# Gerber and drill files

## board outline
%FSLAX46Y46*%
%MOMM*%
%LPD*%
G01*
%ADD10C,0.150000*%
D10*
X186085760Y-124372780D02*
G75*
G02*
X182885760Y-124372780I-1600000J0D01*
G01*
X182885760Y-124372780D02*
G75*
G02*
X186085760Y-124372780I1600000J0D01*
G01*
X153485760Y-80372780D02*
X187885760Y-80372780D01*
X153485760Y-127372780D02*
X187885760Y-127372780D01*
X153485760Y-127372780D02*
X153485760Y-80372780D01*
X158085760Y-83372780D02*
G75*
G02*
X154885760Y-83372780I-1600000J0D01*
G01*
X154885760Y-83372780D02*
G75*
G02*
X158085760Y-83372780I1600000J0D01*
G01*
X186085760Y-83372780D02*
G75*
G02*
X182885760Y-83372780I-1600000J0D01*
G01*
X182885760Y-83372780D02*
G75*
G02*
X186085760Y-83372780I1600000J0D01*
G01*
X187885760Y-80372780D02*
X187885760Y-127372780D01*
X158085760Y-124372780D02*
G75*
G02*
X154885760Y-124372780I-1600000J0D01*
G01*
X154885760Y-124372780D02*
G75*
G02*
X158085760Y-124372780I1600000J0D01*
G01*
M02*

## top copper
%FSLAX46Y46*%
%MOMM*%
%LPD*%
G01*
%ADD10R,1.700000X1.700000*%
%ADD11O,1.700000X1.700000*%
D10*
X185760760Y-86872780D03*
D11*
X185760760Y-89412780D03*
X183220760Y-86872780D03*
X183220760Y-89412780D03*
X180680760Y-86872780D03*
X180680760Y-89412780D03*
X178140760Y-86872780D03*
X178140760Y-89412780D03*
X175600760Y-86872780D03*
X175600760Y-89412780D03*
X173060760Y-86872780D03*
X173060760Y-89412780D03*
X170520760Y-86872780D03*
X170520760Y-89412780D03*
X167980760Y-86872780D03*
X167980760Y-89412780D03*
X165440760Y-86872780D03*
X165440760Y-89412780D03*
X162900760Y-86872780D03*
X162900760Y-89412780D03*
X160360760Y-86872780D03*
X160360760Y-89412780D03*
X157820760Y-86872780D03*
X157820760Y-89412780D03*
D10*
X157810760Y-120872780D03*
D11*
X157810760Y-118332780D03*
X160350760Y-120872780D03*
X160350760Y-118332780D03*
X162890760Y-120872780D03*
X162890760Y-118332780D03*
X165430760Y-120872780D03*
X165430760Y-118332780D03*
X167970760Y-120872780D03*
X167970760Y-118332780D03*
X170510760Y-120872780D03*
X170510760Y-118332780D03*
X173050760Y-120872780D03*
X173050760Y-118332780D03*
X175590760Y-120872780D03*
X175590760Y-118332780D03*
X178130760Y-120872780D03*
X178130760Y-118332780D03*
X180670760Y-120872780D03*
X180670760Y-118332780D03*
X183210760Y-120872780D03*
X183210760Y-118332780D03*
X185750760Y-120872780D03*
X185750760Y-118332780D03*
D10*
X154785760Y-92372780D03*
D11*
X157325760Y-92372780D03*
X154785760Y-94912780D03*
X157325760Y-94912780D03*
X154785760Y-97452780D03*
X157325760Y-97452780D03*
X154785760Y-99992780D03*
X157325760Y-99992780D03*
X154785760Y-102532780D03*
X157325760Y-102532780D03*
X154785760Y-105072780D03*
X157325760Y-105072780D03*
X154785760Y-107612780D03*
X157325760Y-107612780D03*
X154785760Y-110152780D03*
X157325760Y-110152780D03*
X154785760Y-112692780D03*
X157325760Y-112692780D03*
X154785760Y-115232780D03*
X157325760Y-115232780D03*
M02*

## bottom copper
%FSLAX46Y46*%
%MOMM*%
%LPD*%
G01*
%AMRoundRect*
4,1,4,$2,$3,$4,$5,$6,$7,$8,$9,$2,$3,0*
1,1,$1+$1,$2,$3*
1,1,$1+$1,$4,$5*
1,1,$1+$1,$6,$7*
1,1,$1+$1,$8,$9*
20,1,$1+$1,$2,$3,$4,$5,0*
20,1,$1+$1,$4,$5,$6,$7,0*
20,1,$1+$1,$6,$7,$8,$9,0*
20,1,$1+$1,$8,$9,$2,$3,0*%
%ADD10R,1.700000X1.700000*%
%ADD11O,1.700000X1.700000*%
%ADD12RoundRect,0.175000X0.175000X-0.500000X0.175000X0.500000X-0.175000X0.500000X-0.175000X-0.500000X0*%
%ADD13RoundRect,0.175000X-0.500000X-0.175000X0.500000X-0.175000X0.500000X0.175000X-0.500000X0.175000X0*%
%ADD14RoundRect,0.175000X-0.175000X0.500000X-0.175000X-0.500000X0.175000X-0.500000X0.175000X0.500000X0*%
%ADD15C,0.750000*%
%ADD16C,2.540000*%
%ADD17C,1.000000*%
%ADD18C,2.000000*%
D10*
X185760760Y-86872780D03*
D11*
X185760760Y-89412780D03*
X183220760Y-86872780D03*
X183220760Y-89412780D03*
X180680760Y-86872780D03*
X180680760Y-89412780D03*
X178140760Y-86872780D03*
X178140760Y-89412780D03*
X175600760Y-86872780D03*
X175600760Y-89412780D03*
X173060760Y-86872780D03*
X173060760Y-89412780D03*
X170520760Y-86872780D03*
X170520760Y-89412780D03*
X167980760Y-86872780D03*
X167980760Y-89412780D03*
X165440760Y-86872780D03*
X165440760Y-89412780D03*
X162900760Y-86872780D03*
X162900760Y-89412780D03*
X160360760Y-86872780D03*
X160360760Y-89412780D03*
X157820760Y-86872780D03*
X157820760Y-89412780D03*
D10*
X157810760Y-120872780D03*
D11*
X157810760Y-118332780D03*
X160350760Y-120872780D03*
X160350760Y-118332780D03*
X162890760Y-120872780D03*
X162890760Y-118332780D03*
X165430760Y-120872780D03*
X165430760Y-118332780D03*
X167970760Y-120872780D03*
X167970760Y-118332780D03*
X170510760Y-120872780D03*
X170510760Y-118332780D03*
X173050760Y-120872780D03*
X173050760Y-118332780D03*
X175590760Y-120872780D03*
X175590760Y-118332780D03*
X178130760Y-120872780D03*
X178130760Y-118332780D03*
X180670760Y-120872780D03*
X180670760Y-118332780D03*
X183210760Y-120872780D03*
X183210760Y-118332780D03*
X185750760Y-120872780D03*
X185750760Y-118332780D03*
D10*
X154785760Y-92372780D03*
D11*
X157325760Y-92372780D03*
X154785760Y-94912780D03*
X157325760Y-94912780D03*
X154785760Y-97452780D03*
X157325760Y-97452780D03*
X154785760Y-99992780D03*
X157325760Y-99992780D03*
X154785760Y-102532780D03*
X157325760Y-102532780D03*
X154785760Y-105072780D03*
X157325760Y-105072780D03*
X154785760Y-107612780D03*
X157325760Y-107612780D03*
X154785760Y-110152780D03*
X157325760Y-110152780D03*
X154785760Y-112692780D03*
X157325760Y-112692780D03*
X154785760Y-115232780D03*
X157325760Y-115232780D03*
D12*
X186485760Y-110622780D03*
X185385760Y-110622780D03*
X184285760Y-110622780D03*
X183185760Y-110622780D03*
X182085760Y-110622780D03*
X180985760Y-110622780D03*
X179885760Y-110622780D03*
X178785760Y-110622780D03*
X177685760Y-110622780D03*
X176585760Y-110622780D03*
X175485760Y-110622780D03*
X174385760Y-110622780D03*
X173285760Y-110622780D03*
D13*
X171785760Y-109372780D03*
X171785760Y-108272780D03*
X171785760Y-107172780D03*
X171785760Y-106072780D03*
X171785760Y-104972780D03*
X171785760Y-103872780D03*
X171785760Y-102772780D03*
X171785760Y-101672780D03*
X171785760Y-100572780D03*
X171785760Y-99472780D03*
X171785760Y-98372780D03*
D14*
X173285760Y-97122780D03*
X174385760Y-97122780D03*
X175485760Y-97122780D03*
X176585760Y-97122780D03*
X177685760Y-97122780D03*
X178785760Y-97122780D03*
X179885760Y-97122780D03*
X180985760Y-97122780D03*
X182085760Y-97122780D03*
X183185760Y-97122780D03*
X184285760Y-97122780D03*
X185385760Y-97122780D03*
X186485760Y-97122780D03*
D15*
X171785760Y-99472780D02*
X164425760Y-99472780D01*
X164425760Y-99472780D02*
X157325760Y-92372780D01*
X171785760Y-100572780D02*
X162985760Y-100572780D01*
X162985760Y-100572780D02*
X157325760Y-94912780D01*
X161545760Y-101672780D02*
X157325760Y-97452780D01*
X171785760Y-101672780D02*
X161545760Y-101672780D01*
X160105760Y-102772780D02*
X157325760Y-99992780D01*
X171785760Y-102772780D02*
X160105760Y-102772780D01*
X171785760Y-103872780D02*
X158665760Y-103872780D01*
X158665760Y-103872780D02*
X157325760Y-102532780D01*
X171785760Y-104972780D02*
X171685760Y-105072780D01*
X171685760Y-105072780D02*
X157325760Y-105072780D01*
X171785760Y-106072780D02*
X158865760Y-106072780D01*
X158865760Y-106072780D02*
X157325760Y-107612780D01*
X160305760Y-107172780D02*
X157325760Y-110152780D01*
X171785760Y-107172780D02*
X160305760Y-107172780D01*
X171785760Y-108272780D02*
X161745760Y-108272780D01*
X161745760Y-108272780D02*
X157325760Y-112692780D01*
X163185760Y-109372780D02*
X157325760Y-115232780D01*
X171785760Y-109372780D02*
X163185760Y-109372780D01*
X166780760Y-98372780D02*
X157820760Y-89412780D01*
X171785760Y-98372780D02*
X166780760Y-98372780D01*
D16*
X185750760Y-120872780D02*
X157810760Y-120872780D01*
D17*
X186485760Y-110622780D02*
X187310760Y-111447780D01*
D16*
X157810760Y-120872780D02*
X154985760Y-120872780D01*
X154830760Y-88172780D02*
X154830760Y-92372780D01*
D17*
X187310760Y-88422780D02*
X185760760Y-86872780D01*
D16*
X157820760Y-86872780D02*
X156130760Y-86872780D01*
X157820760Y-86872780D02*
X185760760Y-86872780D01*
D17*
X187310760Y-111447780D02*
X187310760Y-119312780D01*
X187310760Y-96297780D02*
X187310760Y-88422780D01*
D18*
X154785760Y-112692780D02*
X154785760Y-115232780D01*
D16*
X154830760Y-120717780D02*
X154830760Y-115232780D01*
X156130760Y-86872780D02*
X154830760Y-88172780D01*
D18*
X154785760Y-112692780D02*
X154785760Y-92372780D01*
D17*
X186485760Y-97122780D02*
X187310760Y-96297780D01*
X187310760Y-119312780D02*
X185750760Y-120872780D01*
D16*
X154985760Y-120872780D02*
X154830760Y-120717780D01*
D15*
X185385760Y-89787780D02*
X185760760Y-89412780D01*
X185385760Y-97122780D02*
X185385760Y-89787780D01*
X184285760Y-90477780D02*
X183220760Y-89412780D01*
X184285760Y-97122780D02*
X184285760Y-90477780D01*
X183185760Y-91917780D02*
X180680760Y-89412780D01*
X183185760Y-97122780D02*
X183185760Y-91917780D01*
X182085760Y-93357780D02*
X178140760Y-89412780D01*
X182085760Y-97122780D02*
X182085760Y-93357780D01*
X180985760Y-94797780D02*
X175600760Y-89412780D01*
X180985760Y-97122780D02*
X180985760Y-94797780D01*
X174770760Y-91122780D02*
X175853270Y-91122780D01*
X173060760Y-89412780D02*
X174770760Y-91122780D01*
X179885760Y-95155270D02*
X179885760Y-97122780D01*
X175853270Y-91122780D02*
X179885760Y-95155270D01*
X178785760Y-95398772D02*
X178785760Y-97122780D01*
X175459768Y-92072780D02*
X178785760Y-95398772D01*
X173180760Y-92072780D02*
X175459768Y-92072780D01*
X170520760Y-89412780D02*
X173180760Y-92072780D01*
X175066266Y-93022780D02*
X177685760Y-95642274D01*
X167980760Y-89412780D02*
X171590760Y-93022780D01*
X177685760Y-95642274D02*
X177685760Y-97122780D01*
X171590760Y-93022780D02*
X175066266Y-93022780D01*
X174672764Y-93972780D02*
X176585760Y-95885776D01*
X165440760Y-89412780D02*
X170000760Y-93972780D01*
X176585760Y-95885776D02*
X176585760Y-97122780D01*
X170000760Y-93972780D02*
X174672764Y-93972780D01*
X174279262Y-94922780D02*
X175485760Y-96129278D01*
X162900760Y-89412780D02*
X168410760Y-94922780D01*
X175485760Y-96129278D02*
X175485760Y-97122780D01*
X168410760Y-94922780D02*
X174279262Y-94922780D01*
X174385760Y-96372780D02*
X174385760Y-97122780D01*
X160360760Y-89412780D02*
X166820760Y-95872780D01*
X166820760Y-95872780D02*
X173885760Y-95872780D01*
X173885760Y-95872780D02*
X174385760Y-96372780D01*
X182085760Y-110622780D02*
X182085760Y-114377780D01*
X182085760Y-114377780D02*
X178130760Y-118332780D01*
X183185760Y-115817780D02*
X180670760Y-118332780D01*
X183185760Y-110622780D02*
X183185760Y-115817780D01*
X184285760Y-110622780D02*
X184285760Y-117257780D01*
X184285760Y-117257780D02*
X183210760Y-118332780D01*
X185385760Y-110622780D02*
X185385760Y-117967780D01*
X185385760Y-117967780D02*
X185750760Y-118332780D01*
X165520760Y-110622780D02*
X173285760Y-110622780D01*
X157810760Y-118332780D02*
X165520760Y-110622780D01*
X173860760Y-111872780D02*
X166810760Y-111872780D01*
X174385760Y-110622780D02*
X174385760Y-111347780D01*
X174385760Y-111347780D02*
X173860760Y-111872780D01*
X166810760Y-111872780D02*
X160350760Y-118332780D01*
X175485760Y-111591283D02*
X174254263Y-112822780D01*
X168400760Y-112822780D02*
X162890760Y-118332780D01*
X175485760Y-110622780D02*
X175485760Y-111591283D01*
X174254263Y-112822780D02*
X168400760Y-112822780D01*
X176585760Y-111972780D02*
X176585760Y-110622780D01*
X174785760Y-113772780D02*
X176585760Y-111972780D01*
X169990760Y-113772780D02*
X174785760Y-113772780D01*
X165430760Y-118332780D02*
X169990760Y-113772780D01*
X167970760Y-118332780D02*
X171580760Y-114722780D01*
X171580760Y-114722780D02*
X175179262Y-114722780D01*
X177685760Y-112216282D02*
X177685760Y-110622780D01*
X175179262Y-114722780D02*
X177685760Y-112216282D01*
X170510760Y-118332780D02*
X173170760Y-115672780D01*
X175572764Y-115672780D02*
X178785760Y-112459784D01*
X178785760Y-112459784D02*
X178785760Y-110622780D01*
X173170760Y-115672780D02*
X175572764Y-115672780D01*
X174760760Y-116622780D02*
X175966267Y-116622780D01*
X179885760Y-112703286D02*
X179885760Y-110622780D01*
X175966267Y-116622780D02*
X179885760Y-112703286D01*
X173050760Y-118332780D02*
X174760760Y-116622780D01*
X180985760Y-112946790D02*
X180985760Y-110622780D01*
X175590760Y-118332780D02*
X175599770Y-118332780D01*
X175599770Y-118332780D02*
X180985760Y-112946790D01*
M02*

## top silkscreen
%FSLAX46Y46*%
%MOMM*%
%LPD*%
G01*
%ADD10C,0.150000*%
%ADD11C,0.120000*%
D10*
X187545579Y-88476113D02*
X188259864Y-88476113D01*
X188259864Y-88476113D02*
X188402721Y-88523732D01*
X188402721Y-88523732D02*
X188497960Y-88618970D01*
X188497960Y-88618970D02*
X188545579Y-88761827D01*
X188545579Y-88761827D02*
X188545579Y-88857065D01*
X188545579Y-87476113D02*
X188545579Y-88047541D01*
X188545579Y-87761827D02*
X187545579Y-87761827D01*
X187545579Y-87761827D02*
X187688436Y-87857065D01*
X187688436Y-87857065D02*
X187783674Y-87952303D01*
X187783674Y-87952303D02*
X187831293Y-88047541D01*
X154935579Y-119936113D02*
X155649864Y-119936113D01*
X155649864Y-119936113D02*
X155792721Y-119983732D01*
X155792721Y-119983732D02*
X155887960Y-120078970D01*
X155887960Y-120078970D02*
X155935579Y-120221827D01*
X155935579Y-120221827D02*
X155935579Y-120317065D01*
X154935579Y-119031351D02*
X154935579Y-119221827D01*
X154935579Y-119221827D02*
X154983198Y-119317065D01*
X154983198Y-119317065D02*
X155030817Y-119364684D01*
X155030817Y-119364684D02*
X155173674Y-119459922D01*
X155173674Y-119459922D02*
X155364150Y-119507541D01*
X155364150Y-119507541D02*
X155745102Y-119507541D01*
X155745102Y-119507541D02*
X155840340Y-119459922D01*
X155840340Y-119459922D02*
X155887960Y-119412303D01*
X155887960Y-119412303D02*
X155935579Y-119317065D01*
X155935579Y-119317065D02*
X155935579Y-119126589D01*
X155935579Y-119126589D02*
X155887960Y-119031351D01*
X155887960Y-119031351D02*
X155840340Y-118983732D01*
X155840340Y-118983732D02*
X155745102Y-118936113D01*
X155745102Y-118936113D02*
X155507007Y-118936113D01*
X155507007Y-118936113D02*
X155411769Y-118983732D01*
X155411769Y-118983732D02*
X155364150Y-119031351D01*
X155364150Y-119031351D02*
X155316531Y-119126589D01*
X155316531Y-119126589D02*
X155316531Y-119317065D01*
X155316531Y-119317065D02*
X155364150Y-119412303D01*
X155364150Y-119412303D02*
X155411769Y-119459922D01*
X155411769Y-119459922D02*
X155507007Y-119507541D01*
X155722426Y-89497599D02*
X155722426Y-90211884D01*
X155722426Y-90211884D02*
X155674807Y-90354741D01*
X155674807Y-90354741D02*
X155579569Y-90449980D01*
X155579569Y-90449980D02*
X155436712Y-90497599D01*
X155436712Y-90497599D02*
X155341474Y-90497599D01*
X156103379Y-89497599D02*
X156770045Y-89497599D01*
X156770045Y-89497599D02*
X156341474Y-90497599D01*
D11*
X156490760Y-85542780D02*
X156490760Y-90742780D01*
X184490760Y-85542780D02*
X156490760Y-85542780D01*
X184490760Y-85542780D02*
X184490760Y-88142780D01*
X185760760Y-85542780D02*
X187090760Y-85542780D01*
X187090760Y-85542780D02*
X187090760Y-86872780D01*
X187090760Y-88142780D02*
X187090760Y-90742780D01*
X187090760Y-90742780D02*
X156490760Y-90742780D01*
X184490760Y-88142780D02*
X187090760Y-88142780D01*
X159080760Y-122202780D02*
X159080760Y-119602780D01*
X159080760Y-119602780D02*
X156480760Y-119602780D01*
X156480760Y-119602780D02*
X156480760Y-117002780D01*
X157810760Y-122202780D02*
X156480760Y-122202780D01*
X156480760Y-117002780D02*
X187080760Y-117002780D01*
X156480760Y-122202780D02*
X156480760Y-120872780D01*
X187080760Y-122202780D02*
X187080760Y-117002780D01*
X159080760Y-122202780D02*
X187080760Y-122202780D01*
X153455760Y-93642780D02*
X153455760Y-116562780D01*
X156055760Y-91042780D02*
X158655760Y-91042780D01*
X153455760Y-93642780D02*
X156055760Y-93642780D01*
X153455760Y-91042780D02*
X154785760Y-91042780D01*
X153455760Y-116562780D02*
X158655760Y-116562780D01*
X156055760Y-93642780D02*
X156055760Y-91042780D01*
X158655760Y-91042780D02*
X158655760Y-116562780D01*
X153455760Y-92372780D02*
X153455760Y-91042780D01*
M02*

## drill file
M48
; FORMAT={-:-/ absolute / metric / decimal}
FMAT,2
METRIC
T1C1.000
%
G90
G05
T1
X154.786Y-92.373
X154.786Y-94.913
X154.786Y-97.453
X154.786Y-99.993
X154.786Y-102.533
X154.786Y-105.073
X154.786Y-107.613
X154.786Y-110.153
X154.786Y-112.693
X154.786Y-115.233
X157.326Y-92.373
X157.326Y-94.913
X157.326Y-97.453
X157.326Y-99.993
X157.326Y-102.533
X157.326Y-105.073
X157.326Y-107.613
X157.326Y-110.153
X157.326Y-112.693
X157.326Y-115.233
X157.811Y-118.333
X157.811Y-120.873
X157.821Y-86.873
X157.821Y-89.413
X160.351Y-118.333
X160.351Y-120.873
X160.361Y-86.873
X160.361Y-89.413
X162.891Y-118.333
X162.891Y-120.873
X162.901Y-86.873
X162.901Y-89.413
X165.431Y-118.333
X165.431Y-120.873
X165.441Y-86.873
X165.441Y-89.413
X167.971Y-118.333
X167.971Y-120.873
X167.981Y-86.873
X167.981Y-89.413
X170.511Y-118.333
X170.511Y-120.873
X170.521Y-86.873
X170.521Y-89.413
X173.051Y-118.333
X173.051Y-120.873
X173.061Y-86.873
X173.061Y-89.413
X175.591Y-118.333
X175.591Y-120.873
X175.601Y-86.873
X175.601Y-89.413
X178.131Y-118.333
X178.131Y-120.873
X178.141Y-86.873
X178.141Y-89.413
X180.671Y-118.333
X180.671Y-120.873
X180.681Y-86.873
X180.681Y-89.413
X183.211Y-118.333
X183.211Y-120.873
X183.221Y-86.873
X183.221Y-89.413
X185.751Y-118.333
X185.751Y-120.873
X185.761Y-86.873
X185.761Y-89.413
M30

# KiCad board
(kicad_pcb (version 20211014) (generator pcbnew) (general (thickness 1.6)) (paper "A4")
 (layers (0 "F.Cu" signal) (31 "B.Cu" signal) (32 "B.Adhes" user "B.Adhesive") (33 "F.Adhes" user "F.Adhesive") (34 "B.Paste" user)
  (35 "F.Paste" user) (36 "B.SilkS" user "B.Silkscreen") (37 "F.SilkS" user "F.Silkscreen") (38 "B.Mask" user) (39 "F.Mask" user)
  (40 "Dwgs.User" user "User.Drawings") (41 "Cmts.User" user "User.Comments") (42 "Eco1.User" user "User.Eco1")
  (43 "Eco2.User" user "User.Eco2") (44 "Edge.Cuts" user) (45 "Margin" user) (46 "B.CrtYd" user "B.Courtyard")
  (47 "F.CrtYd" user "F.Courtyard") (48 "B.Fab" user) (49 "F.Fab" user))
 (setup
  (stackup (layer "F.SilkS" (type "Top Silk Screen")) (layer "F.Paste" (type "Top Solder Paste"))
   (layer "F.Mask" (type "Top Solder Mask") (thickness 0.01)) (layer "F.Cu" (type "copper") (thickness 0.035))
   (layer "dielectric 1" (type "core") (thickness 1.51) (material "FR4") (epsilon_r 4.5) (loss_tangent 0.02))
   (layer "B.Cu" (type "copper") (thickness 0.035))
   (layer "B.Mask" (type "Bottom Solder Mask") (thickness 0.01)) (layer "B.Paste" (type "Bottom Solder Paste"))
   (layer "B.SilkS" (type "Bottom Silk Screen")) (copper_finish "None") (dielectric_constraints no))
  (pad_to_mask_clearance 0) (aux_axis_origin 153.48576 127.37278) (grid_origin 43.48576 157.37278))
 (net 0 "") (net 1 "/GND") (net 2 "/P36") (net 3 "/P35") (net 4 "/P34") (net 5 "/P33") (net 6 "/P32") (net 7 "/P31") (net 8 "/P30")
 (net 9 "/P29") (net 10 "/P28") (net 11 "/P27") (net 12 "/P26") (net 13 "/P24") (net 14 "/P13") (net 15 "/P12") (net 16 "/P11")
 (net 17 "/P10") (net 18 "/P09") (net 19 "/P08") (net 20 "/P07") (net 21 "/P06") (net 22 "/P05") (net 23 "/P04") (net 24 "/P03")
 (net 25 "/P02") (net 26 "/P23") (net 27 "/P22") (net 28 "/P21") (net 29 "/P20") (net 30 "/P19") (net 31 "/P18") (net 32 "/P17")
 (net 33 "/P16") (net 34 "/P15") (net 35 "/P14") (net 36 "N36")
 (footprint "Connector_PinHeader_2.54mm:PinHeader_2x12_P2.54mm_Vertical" (layer "F.Cu") (at 185.76076 86.87278 -90)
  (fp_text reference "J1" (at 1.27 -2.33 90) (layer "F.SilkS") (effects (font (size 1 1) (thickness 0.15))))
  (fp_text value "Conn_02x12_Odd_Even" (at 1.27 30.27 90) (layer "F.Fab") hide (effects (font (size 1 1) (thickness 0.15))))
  (fp_line (start -1.33 29.27) (end 3.87 29.27) (layer "F.SilkS") (width 0.12))
  (fp_line (start -1.33 1.27) (end -1.33 29.27) (layer "F.SilkS") (width 0.12))
  (fp_line (start -1.33 1.27) (end 1.27 1.27) (layer "F.SilkS") (width 0.12))
  (fp_line (start -1.33 0) (end -1.33 -1.33) (layer "F.SilkS") (width 0.12))
  (fp_line (start -1.33 -1.33) (end 0 -1.33) (layer "F.SilkS") (width 0.12))
  (fp_line (start 1.27 -1.33) (end 3.87 -1.33) (layer "F.SilkS") (width 0.12))
  (fp_line (start 3.87 -1.33) (end 3.87 29.27) (layer "F.SilkS") (width 0.12))
  (fp_line (start 1.27 1.27) (end 1.27 -1.33) (layer "F.SilkS") (width 0.12))
  (pad "1" thru_hole rect (at 0 0 270) (size 1.7 1.7) (drill 1) (layers *.Cu *.Mask) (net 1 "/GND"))
  (pad "2" thru_hole oval (at 2.54 0 270) (size 1.7 1.7) (drill 1) (layers *.Cu *.Mask) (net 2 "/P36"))
  (pad "3" thru_hole oval (at 0 2.54 270) (size 1.7 1.7) (drill 1) (layers *.Cu *.Mask) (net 1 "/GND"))
  (pad "4" thru_hole oval (at 2.54 2.54 270) (size 1.7 1.7) (drill 1) (layers *.Cu *.Mask) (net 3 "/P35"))
  (pad "5" thru_hole oval (at 0 5.08 270) (size 1.7 1.7) (drill 1) (layers *.Cu *.Mask) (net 1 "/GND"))
  (pad "6" thru_hole oval (at 2.54 5.08 270) (size 1.7 1.7) (drill 1) (layers *.Cu *.Mask) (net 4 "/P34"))
  (pad "7" thru_hole oval (at 0 7.62 270) (size 1.7 1.7) (drill 1) (layers *.Cu *.Mask) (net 1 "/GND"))
  (pad "8" thru_hole oval (at 2.54 7.62 270) (size 1.7 1.7) (drill 1) (layers *.Cu *.Mask) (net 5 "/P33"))
  (pad "9" thru_hole oval (at 0 10.16 270) (size 1.7 1.7) (drill 1) (layers *.Cu *.Mask) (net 1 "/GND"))
  (pad "10" thru_hole oval (at 2.54 10.16 270) (size 1.7 1.7) (drill 1) (layers *.Cu *.Mask) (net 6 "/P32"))
  (pad "11" thru_hole oval (at 0 12.7 270) (size 1.7 1.7) (drill 1) (layers *.Cu *.Mask) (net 1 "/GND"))
  (pad "12" thru_hole oval (at 2.54 12.7 270) (size 1.7 1.7) (drill 1) (layers *.Cu *.Mask) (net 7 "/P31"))
  (pad "13" thru_hole oval (at 0 15.24 270) (size 1.7 1.7) (drill 1) (layers *.Cu *.Mask) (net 1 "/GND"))
  (pad "14" thru_hole oval (at 2.54 15.24 270) (size 1.7 1.7) (drill 1) (layers *.Cu *.Mask) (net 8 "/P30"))
  (pad "15" thru_hole oval (at 0 17.78 270) (size 1.7 1.7) (drill 1) (layers *.Cu *.Mask) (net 1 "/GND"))
  (pad "16" thru_hole oval (at 2.54 17.78 270) (size 1.7 1.7) (drill 1) (layers *.Cu *.Mask) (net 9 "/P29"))
  (pad "17" thru_hole oval (at 0 20.32 270) (size 1.7 1.7) (drill 1) (layers *.Cu *.Mask) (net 1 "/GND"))
  (pad "18" thru_hole oval (at 2.54 20.32 270) (size 1.7 1.7) (drill 1) (layers *.Cu *.Mask) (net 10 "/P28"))
  (pad "19" thru_hole oval (at 0 22.86 270) (size 1.7 1.7) (drill 1) (layers *.Cu *.Mask) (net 1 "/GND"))
  (pad "20" thru_hole oval (at 2.54 22.86 270) (size 1.7 1.7) (drill 1) (layers *.Cu *.Mask) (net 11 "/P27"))
  (pad "21" thru_hole oval (at 0 25.4 270) (size 1.7 1.7) (drill 1) (layers *.Cu *.Mask) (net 1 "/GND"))
  (pad "22" thru_hole oval (at 2.54 25.4 270) (size 1.7 1.7) (drill 1) (layers *.Cu *.Mask) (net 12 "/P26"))
  (pad "23" thru_hole oval (at 0 27.94 270) (size 1.7 1.7) (drill 1) (layers *.Cu *.Mask) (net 1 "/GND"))
  (pad "24" thru_hole oval (at 2.54 27.94 270) (size 1.7 1.7) (drill 1) (layers *.Cu *.Mask) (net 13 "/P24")))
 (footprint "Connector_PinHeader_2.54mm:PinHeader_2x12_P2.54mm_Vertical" (layer "F.Cu") (at 157.81076 120.87278 90)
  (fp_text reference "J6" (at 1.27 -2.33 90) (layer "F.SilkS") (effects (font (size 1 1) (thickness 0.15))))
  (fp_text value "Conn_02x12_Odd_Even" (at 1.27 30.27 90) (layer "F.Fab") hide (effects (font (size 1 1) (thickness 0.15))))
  (fp_line (start -1.33 1.27) (end 1.27 1.27) (layer "F.SilkS") (width 0.12))
  (fp_line (start 1.27 1.27) (end 1.27 -1.33) (layer "F.SilkS") (width 0.12))
  (fp_line (start 1.27 -1.33) (end 3.87 -1.33) (layer "F.SilkS") (width 0.12))
  (fp_line (start -1.33 0) (end -1.33 -1.33) (layer "F.SilkS") (width 0.12))
  (fp_line (start 3.87 -1.33) (end 3.87 29.27) (layer "F.SilkS") (width 0.12))
  (fp_line (start -1.33 -1.33) (end 0 -1.33) (layer "F.SilkS") (width 0.12))
  (fp_line (start -1.33 29.27) (end 3.87 29.27) (layer "F.SilkS") (width 0.12))
  (fp_line (start -1.33 1.27) (end -1.33 29.27) (layer "F.SilkS") (width 0.12))
  (pad "1" thru_hole rect (at 0 0 90) (size 1.7 1.7) (drill 1) (layers *.Cu *.Mask) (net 1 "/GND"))
  (pad "2" thru_hole oval (at 2.54 0 90) (size 1.7 1.7) (drill 1) (layers *.Cu *.Mask) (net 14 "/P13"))
  (pad "3" thru_hole oval (at 0 2.54 90) (size 1.7 1.7) (drill 1) (layers *.Cu *.Mask) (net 1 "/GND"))
  (pad "4" thru_hole oval (at 2.54 2.54 90) (size 1.7 1.7) (drill 1) (layers *.Cu *.Mask) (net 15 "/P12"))
  (pad "5" thru_hole oval (at 0 5.08 90) (size 1.7 1.7) (drill 1) (layers *.Cu *.Mask) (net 1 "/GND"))
  (pad "6" thru_hole oval (at 2.54 5.08 90) (size 1.7 1.7) (drill 1) (layers *.Cu *.Mask) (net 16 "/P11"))
  (pad "7" thru_hole oval (at 0 7.62 90) (size 1.7 1.7) (drill 1) (layers *.Cu *.Mask) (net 1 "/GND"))
  (pad "8" thru_hole oval (at 2.54 7.62 90) (size 1.7 1.7) (drill 1) (layers *.Cu *.Mask) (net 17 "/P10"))
  (pad "9" thru_hole oval (at 0 10.16 90) (size 1.7 1.7) (drill 1) (layers *.Cu *.Mask) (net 1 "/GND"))
  (pad "10" thru_hole oval (at 2.54 10.16 90) (size 1.7 1.7) (drill 1) (layers *.Cu *.Mask) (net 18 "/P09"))
  (pad "11" thru_hole oval (at 0 12.7 90) (size 1.7 1.7) (drill 1) (layers *.Cu *.Mask) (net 1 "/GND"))
  (pad "12" thru_hole oval (at 2.54 12.7 90) (size 1.7 1.7) (drill 1) (layers *.Cu *.Mask) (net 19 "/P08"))
  (pad "13" thru_hole oval (at 0 15.24 90) (size 1.7 1.7) (drill 1) (layers *.Cu *.Mask) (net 1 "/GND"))
  (pad "14" thru_hole oval (at 2.54 15.24 90) (size 1.7 1.7) (drill 1) (layers *.Cu *.Mask) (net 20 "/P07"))
  (pad "15" thru_hole oval (at 0 17.78 90) (size 1.7 1.7) (drill 1) (layers *.Cu *.Mask) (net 1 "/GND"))
  (pad "16" thru_hole oval (at 2.54 17.78 90) (size 1.7 1.7) (drill 1) (layers *.Cu *.Mask) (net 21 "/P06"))
  (pad "17" thru_hole oval (at 0 20.32 90) (size 1.7 1.7) (drill 1) (layers *.Cu *.Mask) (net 1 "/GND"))
  (pad "18" thru_hole oval (at 2.54 20.32 90) (size 1.7 1.7) (drill 1) (layers *.Cu *.Mask) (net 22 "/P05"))
  (pad "19" thru_hole oval (at 0 22.86 90) (size 1.7 1.7) (drill 1) (layers *.Cu *.Mask) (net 1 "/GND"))
  (pad "20" thru_hole oval (at 2.54 22.86 90) (size 1.7 1.7) (drill 1) (layers *.Cu *.Mask) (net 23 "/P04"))
  (pad "21" thru_hole oval (at 0 25.4 90) (size 1.7 1.7) (drill 1) (layers *.Cu *.Mask) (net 1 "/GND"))
  (pad "22" thru_hole oval (at 2.54 25.4 90) (size 1.7 1.7) (drill 1) (layers *.Cu *.Mask) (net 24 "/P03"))
  (pad "23" thru_hole oval (at 0 27.94 90) (size 1.7 1.7) (drill 1) (layers *.Cu *.Mask) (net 1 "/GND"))
  (pad "24" thru_hole oval (at 2.54 27.94 90) (size 1.7 1.7) (drill 1) (layers *.Cu *.Mask) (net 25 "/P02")))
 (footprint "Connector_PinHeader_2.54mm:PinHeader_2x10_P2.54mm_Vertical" (layer "F.Cu") (at 154.78576 92.37278)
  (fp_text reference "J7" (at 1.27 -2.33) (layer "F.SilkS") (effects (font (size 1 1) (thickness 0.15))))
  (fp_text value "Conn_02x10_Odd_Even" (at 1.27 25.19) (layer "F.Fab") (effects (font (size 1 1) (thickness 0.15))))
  (fp_line (start -1.33 1.27) (end -1.33 24.19) (layer "F.SilkS") (width 0.12))
  (fp_line (start 1.27 -1.33) (end 3.87 -1.33) (layer "F.SilkS") (width 0.12))
  (fp_line (start -1.33 1.27) (end 1.27 1.27) (layer "F.SilkS") (width 0.12))
  (fp_line (start -1.33 -1.33) (end 0 -1.33) (layer "F.SilkS") (width 0.12))
  (fp_line (start -1.33 24.19) (end 3.87 24.19) (layer "F.SilkS") (width 0.12))
  (fp_line (start 1.27 1.27) (end 1.27 -1.33) (layer "F.SilkS") (width 0.12))
  (fp_line (start 3.87 -1.33) (end 3.87 24.19) (layer "F.SilkS") (width 0.12))
  (fp_line (start -1.33 0) (end -1.33 -1.33) (layer "F.SilkS") (width 0.12))
  (pad "1" thru_hole rect (at 0 0) (size 1.7 1.7) (drill 1) (layers *.Cu *.Mask) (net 1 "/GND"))
  (pad "2" thru_hole oval (at 2.54 0) (size 1.7 1.7) (drill 1) (layers *.Cu *.Mask) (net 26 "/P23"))
  (pad "3" thru_hole oval (at 0 2.54) (size 1.7 1.7) (drill 1) (layers *.Cu *.Mask) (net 1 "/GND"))
  (pad "4" thru_hole oval (at 2.54 2.54) (size 1.7 1.7) (drill 1) (layers *.Cu *.Mask) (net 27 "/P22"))
  (pad "5" thru_hole oval (at 0 5.08) (size 1.7 1.7) (drill 1) (layers *.Cu *.Mask) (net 1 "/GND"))
  (pad "6" thru_hole oval (at 2.54 5.08) (size 1.7 1.7) (drill 1) (layers *.Cu *.Mask) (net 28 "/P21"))
  (pad "7" thru_hole oval (at 0 7.62) (size 1.7 1.7) (drill 1) (layers *.Cu *.Mask) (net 1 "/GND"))
  (pad "8" thru_hole oval (at 2.54 7.62) (size 1.7 1.7) (drill 1) (layers *.Cu *.Mask) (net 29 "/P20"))
  (pad "9" thru_hole oval (at 0 10.16) (size 1.7 1.7) (drill 1) (layers *.Cu *.Mask) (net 1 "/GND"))
  (pad "10" thru_hole oval (at 2.54 10.16) (size 1.7 1.7) (drill 1) (layers *.Cu *.Mask) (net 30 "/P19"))
  (pad "11" thru_hole oval (at 0 12.7) (size 1.7 1.7) (drill 1) (layers *.Cu *.Mask) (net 1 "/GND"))
  (pad "12" thru_hole oval (at 2.54 12.7) (size 1.7 1.7) (drill 1) (layers *.Cu *.Mask) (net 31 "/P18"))
  (pad "13" thru_hole oval (at 0 15.24) (size 1.7 1.7) (drill 1) (layers *.Cu *.Mask) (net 1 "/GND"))
  (pad "14" thru_hole oval (at 2.54 15.24) (size 1.7 1.7) (drill 1) (layers *.Cu *.Mask) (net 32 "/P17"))
  (pad "15" thru_hole oval (at 0 17.78) (size 1.7 1.7) (drill 1) (layers *.Cu *.Mask) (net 1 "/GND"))
  (pad "16" thru_hole oval (at 2.54 17.78) (size 1.7 1.7) (drill 1) (layers *.Cu *.Mask) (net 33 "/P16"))
  (pad "17" thru_hole oval (at 0 20.32) (size 1.7 1.7) (drill 1) (layers *.Cu *.Mask) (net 1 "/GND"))
  (pad "18" thru_hole oval (at 2.54 20.32) (size 1.7 1.7) (drill 1) (layers *.Cu *.Mask) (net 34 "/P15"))
  (pad "19" thru_hole oval (at 0 22.86) (size 1.7 1.7) (drill 1) (layers *.Cu *.Mask) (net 1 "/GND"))
  (pad "20" thru_hole oval (at 2.54 22.86) (size 1.7 1.7) (drill 1) (layers *.Cu *.Mask) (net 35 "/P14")))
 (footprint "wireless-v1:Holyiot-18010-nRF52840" (layer "B.Cu") (at 180.78576 103.87278 90)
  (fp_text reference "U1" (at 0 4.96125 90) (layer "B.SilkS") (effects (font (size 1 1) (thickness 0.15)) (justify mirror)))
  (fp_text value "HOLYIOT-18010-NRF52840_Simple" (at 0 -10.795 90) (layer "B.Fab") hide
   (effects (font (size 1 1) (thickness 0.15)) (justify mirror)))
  (pad "1" smd roundrect (at -6.75 5.7 90) (size 1.35 0.7) (layers "B.Cu" "B.Paste" "B.Mask") (roundrect_rratio 0.25) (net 1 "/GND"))
  (pad "2" smd roundrect (at -6.75 4.6 90) (size 1.35 0.7) (layers "B.Cu" "B.Paste" "B.Mask") (roundrect_rratio 0.25) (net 25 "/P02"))
  (pad "3" smd roundrect (at -6.75 3.5 90) (size 1.35 0.7) (layers "B.Cu" "B.Paste" "B.Mask") (roundrect_rratio 0.25) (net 24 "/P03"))
  (pad "4" smd roundrect (at -6.75 2.4 90) (size 1.35 0.7) (layers "B.Cu" "B.Paste" "B.Mask") (roundrect_rratio 0.25) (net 23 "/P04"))
  (pad "5" smd roundrect (at -6.75 1.3 90) (size 1.35 0.7) (layers "B.Cu" "B.Paste" "B.Mask") (roundrect_rratio 0.25) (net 22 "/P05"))
  (pad "6" smd roundrect (at -6.75 0.2 90) (size 1.35 0.7) (layers "B.Cu" "B.Paste" "B.Mask") (roundrect_rratio 0.25) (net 21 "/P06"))
  (pad "7" smd roundrect (at -6.75 -0.9 90) (size 1.35 0.7) (layers "B.Cu" "B.Paste" "B.Mask") (roundrect_rratio 0.25) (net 20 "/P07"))
  (pad "8" smd roundrect (at -6.75 -2 90) (size 1.35 0.7) (layers "B.Cu" "B.Paste" "B.Mask") (roundrect_rratio 0.25) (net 19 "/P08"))
  (pad "9" smd roundrect (at -6.75 -3.1 90) (size 1.35 0.7) (layers "B.Cu" "B.Paste" "B.Mask") (roundrect_rratio 0.25) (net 18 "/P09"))
  (pad "10" smd roundrect (at -6.75 -4.2 90) (size 1.35 0.7) (layers "B.Cu" "B.Paste" "B.Mask") (roundrect_rratio 0.25) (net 17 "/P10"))
  (pad "11" smd roundrect (at -6.75 -5.3 90) (size 1.35 0.7) (layers "B.Cu" "B.Paste" "B.Mask") (roundrect_rratio 0.25) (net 16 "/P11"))
  (pad "12" smd roundrect (at -6.75 -6.4 90) (size 1.35 0.7) (layers "B.Cu" "B.Paste" "B.Mask") (roundrect_rratio 0.25) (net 15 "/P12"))
  (pad "13" smd roundrect (at -6.75 -7.5 90) (size 1.35 0.7) (layers "B.Cu" "B.Paste" "B.Mask") (roundrect_rratio 0.25) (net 14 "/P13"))
  (pad "14" smd roundrect (at -5.5 -9) (size 1.35 0.7) (layers "B.Cu" "B.Paste" "B.Mask") (roundrect_rratio 0.25) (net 35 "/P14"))
  (pad "15" smd roundrect (at -4.4 -9) (size 1.35 0.7) (layers "B.Cu" "B.Paste" "B.Mask") (roundrect_rratio 0.25) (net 34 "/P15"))
  (pad "16" smd roundrect (at -3.3 -9) (size 1.35 0.7) (layers "B.Cu" "B.Paste" "B.Mask") (roundrect_rratio 0.25) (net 33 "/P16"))
  (pad "17" smd roundrect (at -2.2 -9) (size 1.35 0.7) (layers "B.Cu" "B.Paste" "B.Mask") (roundrect_rratio 0.25) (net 32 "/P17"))
  (pad "18" smd roundrect (at -1.1 -9) (size 1.35 0.7) (layers "B.Cu" "B.Paste" "B.Mask") (roundrect_rratio 0.25) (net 31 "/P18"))
  (pad "19" smd roundrect (at 0 -9) (size 1.35 0.7) (layers "B.Cu" "B.Paste" "B.Mask") (roundrect_rratio 0.25) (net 30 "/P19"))
  (pad "20" smd roundrect (at 1.1 -9) (size 1.35 0.7) (layers "B.Cu" "B.Paste" "B.Mask") (roundrect_rratio 0.25) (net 29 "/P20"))
  (pad "21" smd roundrect (at 2.2 -9) (size 1.35 0.7) (layers "B.Cu" "B.Paste" "B.Mask") (roundrect_rratio 0.25) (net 28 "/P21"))
  (pad "22" smd roundrect (at 3.3 -9) (size 1.35 0.7) (layers "B.Cu" "B.Paste" "B.Mask") (roundrect_rratio 0.25) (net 27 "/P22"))
  (pad "23" smd roundrect (at 4.4 -9) (size 1.35 0.7) (layers "B.Cu" "B.Paste" "B.Mask") (roundrect_rratio 0.25) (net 26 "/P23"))
  (pad "24" smd roundrect (at 5.5 -9) (size 1.35 0.7) (layers "B.Cu" "B.Paste" "B.Mask") (roundrect_rratio 0.25) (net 13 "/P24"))
  (pad "25" smd roundrect (at 6.75 -7.5 270) (size 1.35 0.7) (layers "B.Cu" "B.Paste" "B.Mask") (roundrect_rratio 0.25) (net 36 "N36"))
  (pad "26" smd roundrect (at 6.75 -6.4 270) (size 1.35 0.7) (layers "B.Cu" "B.Paste" "B.Mask") (roundrect_rratio 0.25) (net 12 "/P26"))
  (pad "27" smd roundrect (at 6.75 -5.3 270) (size 1.35 0.7) (layers "B.Cu" "B.Paste" "B.Mask") (roundrect_rratio 0.25) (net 11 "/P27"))
  (pad "28" smd roundrect (at 6.75 -4.2 270) (size 1.35 0.7) (layers "B.Cu" "B.Paste" "B.Mask") (roundrect_rratio 0.25) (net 10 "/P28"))
  (pad "29" smd roundrect (at 6.75 -3.1 270) (size 1.35 0.7) (layers "B.Cu" "B.Paste" "B.Mask") (roundrect_rratio 0.25) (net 9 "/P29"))
  (pad "30" smd roundrect (at 6.75 -2 270) (size 1.35 0.7) (layers "B.Cu" "B.Paste" "B.Mask") (roundrect_rratio 0.25) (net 8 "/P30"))
  (pad "31" smd roundrect (at 6.75 -0.9 270) (size 1.35 0.7) (layers "B.Cu" "B.Paste" "B.Mask") (roundrect_rratio 0.25) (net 7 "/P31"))
  (pad "32" smd roundrect (at 6.75 0.2 270) (size 1.35 0.7) (layers "B.Cu" "B.Paste" "B.Mask") (roundrect_rratio 0.25) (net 6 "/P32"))
  (pad "33" smd roundrect (at 6.75 1.3 270) (size 1.35 0.7) (layers "B.Cu" "B.Paste" "B.Mask") (roundrect_rratio 0.25) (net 5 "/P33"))
  (pad "34" smd roundrect (at 6.75 2.4 270) (size 1.35 0.7) (layers "B.Cu" "B.Paste" "B.Mask") (roundrect_rratio 0.25) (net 4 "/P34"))
  (pad "35" smd roundrect (at 6.75 3.5 270) (size 1.35 0.7) (layers "B.Cu" "B.Paste" "B.Mask") (roundrect_rratio 0.25) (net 3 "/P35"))
  (pad "36" smd roundrect (at 6.75 4.6 270) (size 1.35 0.7) (layers "B.Cu" "B.Paste" "B.Mask") (roundrect_rratio 0.25) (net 2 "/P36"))
  (pad "37" smd roundrect (at 6.75 5.7 270) (size 1.35 0.7) (layers "B.Cu" "B.Paste" "B.Mask") (roundrect_rratio 0.25) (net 1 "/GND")))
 (gr_circle (center 184.48576 124.37278) (end 186.08576 124.37278) (layer "Edge.Cuts") (width 0.15) (fill none))
 (gr_line (start 153.48576 80.37278) (end 187.88576 80.37278) (layer "Edge.Cuts") (width 0.15))
 (gr_line (start 153.48576 127.37278) (end 187.88576 127.37278) (layer "Edge.Cuts") (width 0.15))
 (gr_line (start 153.48576 127.37278) (end 153.48576 80.37278) (layer "Edge.Cuts") (width 0.15))
 (gr_circle (center 156.48576 83.37278) (end 158.08576 83.37278) (layer "Edge.Cuts") (width 0.15) (fill none))
 (gr_circle (center 184.48576 83.37278) (end 186.08576 83.37278) (layer "Edge.Cuts") (width 0.15) (fill none))
 (gr_line (start 187.88576 80.37278) (end 187.88576 127.37278) (layer "Edge.Cuts") (width 0.15))
 (gr_circle (center 156.48576 124.37278) (end 158.08576 124.37278) (layer "Edge.Cuts") (width 0.15) (fill none))
 (segment (start 171.78576 99.47278) (end 164.42576 99.47278) (width 0.75) (layer "B.Cu") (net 26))
 (segment (start 164.42576 99.47278) (end 157.32576 92.37278) (width 0.75) (layer "B.Cu") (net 26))
 (segment (start 171.78576 100.57278) (end 162.98576 100.57278) (width 0.75) (layer "B.Cu") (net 27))
 (segment (start 162.98576 100.57278) (end 157.32576 94.91278) (width 0.75) (layer "B.Cu") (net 27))
 (segment (start 161.54576 101.67278) (end 157.32576 97.45278) (width 0.75) (layer "B.Cu") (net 28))
 (segment (start 171.78576 101.67278) (end 161.54576 101.67278) (width 0.75) (layer "B.Cu") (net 28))
 (segment (start 160.10576 102.77278) (end 157.32576 99.99278) (width 0.75) (layer "B.Cu") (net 29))
 (segment (start 171.78576 102.77278) (end 160.10576 102.77278) (width 0.75) (layer "B.Cu") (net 29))
 (segment (start 171.78576 103.87278) (end 158.66576 103.87278) (width 0.75) (layer "B.Cu") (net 30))
 (segment (start 158.66576 103.87278) (end 157.32576 102.53278) (width 0.75) (layer "B.Cu") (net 30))
 (segment (start 171.78576 104.97278) (end 171.68576 105.07278) (width 0.75) (layer "B.Cu") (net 31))
 (segment (start 171.68576 105.07278) (end 157.32576 105.07278) (width 0.75) (layer "B.Cu") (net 31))
 (segment (start 171.78576 106.07278) (end 158.86576 106.07278) (width 0.75) (layer "B.Cu") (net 32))
 (segment (start 158.86576 106.07278) (end 157.32576 107.61278) (width 0.75) (layer "B.Cu") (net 32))
 (segment (start 160.30576 107.17278) (end 157.32576 110.15278) (width 0.75) (layer "B.Cu") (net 33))
 (segment (start 171.78576 107.17278) (end 160.30576 107.17278) (width 0.75) (layer "B.Cu") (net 33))
 (segment (start 171.78576 108.27278) (end 161.74576 108.27278) (width 0.75) (layer "B.Cu") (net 34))
 (segment (start 161.74576 108.27278) (end 157.32576 112.69278) (width 0.75) (layer "B.Cu") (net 34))
 (segment (start 163.18576 109.37278) (end 157.32576 115.23278) (width 0.75) (layer "B.Cu") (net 35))
 (segment (start 171.78576 109.37278) (end 163.18576 109.37278) (width 0.75) (layer "B.Cu") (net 35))
 (segment (start 166.78076 98.37278) (end 157.82076 89.41278) (width 0.75) (layer "B.Cu") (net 13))
 (segment (start 171.78576 98.37278) (end 166.78076 98.37278) (width 0.75) (layer "B.Cu") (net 13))
 (segment (start 185.75076 120.87278) (end 157.81076 120.87278) (width 2.54) (layer "B.Cu") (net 1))
 (segment (start 186.48576 110.62278) (end 187.31076 111.44778) (width 1) (layer "B.Cu") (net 1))
 (segment (start 157.81076 120.87278) (end 154.98576 120.87278) (width 2.54) (layer "B.Cu") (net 1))
 (segment (start 154.83076 88.17278) (end 154.83076 92.37278) (width 2.54) (layer "B.Cu") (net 1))
 (segment (start 187.31076 88.42278) (end 185.76076 86.87278) (width 1) (layer "B.Cu") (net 1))
 (segment (start 157.82076 86.87278) (end 156.13076 86.87278) (width 2.54) (layer "B.Cu") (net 1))
 (segment (start 157.82076 86.87278) (end 185.76076 86.87278) (width 2.54) (layer "B.Cu") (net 1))
 (segment (start 187.31076 111.44778) (end 187.31076 119.31278) (width 1) (layer "B.Cu") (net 1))
 (segment (start 187.31076 96.29778) (end 187.31076 88.42278) (width 1) (layer "B.Cu") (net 1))
 (segment (start 154.78576 112.69278) (end 154.78576 115.23278) (width 2) (layer "B.Cu") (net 1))
 (segment (start 154.83076 120.71778) (end 154.83076 115.23278) (width 2.54) (layer "B.Cu") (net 1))
 (segment (start 156.13076 86.87278) (end 154.83076 88.17278) (width 2.54) (layer "B.Cu") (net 1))
 (segment (start 154.78576 112.69278) (end 154.78576 92.37278) (width 2) (layer "B.Cu") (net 1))
 (segment (start 186.48576 97.12278) (end 187.31076 96.29778) (width 1) (layer "B.Cu") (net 1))
 (segment (start 187.31076 119.31278) (end 185.75076 120.87278) (width 1) (layer "B.Cu") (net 1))
 (segment (start 154.98576 120.87278) (end 154.83076 120.71778) (width 2.54) (layer "B.Cu") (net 1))
 (segment (start 185.38576 89.78778) (end 185.76076 89.41278) (width 0.75) (layer "B.Cu") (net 2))
 (segment (start 185.38576 97.12278) (end 185.38576 89.78778) (width 0.75) (layer "B.Cu") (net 2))
 (segment (start 184.28576 90.47778) (end 183.22076 89.41278) (width 0.75) (layer "B.Cu") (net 3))
 (segment (start 184.28576 97.12278) (end 184.28576 90.47778) (width 0.75) (layer "B.Cu") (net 3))
 (segment (start 183.18576 91.91778) (end 180.68076 89.41278) (width 0.75) (layer "B.Cu") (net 4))
 (segment (start 183.18576 97.12278) (end 183.18576 91.91778) (width 0.75) (layer "B.Cu") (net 4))
 (segment (start 182.08576 93.35778) (end 178.14076 89.41278) (width 0.75) (layer "B.Cu") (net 5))
 (segment (start 182.08576 97.12278) (end 182.08576 93.35778) (width 0.75) (layer "B.Cu") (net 5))
 (segment (start 180.98576 94.79778) (end 175.60076 89.41278) (width 0.75) (layer "B.Cu") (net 6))
 (segment (start 180.98576 97.12278) (end 180.98576 94.79778) (width 0.75) (layer "B.Cu") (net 6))
 (segment (start 174.77076 91.12278) (end 175.85327 91.12278) (width 0.75) (layer "B.Cu") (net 7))
 (segment (start 173.06076 89.41278) (end 174.77076 91.12278) (width 0.75) (layer "B.Cu") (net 7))
 (segment (start 179.88576 95.15527) (end 179.88576 97.12278) (width 0.75) (layer "B.Cu") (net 7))
 (segment (start 175.85327 91.12278) (end 179.88576 95.15527) (width 0.75) (layer "B.Cu") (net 7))
 (segment (start 178.78576 95.398772) (end 178.78576 97.12278) (width 0.75) (layer "B.Cu") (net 8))
 (segment (start 175.459768 92.07278) (end 178.78576 95.398772) (width 0.75) (layer "B.Cu") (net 8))
 (segment (start 173.18076 92.07278) (end 175.459768 92.07278) (width 0.75) (layer "B.Cu") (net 8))
 (segment (start 170.52076 89.41278) (end 173.18076 92.07278) (width 0.75) (layer "B.Cu") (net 8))
 (segment (start 175.066266 93.02278) (end 177.68576 95.642274) (width 0.75) (layer "B.Cu") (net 9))
 (segment (start 167.98076 89.41278) (end 171.59076 93.02278) (width 0.75) (layer "B.Cu") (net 9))
 (segment (start 177.68576 95.642274) (end 177.68576 97.12278) (width 0.75) (layer "B.Cu") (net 9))
 (segment (start 171.59076 93.02278) (end 175.066266 93.02278) (width 0.75) (layer "B.Cu") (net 9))
 (segment (start 174.672764 93.97278) (end 176.58576 95.885776) (width 0.75) (layer "B.Cu") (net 10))
 (segment (start 165.44076 89.41278) (end 170.00076 93.97278) (width 0.75) (layer "B.Cu") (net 10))
 (segment (start 176.58576 95.885776) (end 176.58576 97.12278) (width 0.75) (layer "B.Cu") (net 10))
 (segment (start 170.00076 93.97278) (end 174.672764 93.97278) (width 0.75) (layer "B.Cu") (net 10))
 (segment (start 174.279262 94.92278) (end 175.48576 96.129278) (width 0.75) (layer "B.Cu") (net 11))
 (segment (start 162.90076 89.41278) (end 168.41076 94.92278) (width 0.75) (layer "B.Cu") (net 11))
 (segment (start 175.48576 96.129278) (end 175.48576 97.12278) (width 0.75) (layer "B.Cu") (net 11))
 (segment (start 168.41076 94.92278) (end 174.279262 94.92278) (width 0.75) (layer "B.Cu") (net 11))
 (segment (start 174.38576 96.37278) (end 174.38576 97.12278) (width 0.75) (layer "B.Cu") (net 12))
 (segment (start 160.36076 89.41278) (end 166.82076 95.87278) (width 0.75) (layer "B.Cu") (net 12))
 (segment (start 166.82076 95.87278) (end 173.88576 95.87278) (width 0.75) (layer "B.Cu") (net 12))
 (segment (start 173.88576 95.87278) (end 174.38576 96.37278) (width 0.75) (layer "B.Cu") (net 12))
 (segment (start 182.08576 110.62278) (end 182.08576 114.37778) (width 0.75) (layer "B.Cu") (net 22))
 (segment (start 182.08576 114.37778) (end 178.13076 118.33278) (width 0.75) (layer "B.Cu") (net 22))
 (segment (start 183.18576 115.81778) (end 180.67076 118.33278) (width 0.75) (layer "B.Cu") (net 23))
 (segment (start 183.18576 110.62278) (end 183.18576 115.81778) (width 0.75) (layer "B.Cu") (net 23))
 (segment (start 184.28576 110.62278) (end 184.28576 117.25778) (width 0.75) (layer "B.Cu") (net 24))
 (segment (start 184.28576 117.25778) (end 183.21076 118.33278) (width 0.75) (layer "B.Cu") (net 24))
 (segment (start 185.38576 110.62278) (end 185.38576 117.96778) (width 0.75) (layer "B.Cu") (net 25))
 (segment (start 185.38576 117.96778) (end 185.75076 118.33278) (width 0.75) (layer "B.Cu") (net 25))
 (segment (start 165.52076 110.62278) (end 173.28576 110.62278) (width 0.75) (layer "B.Cu") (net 14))
 (segment (start 157.81076 118.33278) (end 165.52076 110.62278) (width 0.75) (layer "B.Cu") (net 14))
 (segment (start 173.86076 111.87278) (end 166.81076 111.87278) (width 0.75) (layer "B.Cu") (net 15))
 (segment (start 174.38576 110.62278) (end 174.38576 111.34778) (width 0.75) (layer "B.Cu") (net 15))
 (segment (start 174.38576 111.34778) (end 173.86076 111.87278) (width 0.75) (layer "B.Cu") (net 15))
 (segment (start 166.81076 111.87278) (end 160.35076 118.33278) (width 0.75) (layer "B.Cu") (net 15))
 (segment (start 175.48576 111.591283) (end 174.254263 112.82278) (width 0.75) (layer "B.Cu") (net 16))
 (segment (start 168.40076 112.82278) (end 162.89076 118.33278) (width 0.75) (layer "B.Cu") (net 16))
 (segment (start 175.48576 110.62278) (end 175.48576 111.591283) (width 0.75) (layer "B.Cu") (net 16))
 (segment (start 174.254263 112.82278) (end 168.40076 112.82278) (width 0.75) (layer "B.Cu") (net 16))
 (segment (start 176.58576 111.97278) (end 176.58576 110.62278) (width 0.75) (layer "B.Cu") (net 17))
 (segment (start 174.78576 113.77278) (end 176.58576 111.97278) (width 0.75) (layer "B.Cu") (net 17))
 (segment (start 169.99076 113.77278) (end 174.78576 113.77278) (width 0.75) (layer "B.Cu") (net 17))
 (segment (start 165.43076 118.33278) (end 169.99076 113.77278) (width 0.75) (layer "B.Cu") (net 17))
 (segment (start 167.97076 118.33278) (end 171.58076 114.72278) (width 0.75) (layer "B.Cu") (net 18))
 (segment (start 171.58076 114.72278) (end 175.179262 114.72278) (width 0.75) (layer "B.Cu") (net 18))
 (segment (start 177.68576 112.216282) (end 177.68576 110.62278) (width 0.75) (layer "B.Cu") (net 18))
 (segment (start 175.179262 114.72278) (end 177.68576 112.216282) (width 0.75) (layer "B.Cu") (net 18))
 (segment (start 170.51076 118.33278) (end 173.17076 115.67278) (width 0.75) (layer "B.Cu") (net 19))
 (segment (start 175.572764 115.67278) (end 178.78576 112.459784) (width 0.75) (layer "B.Cu") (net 19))
 (segment (start 178.78576 112.459784) (end 178.78576 110.62278) (width 0.75) (layer "B.Cu") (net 19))
 (segment (start 173.17076 115.67278) (end 175.572764 115.67278) (width 0.75) (layer "B.Cu") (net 19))
 (segment (start 174.76076 116.62278) (end 175.966267 116.62278) (width 0.75) (layer "B.Cu") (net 20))
 (segment (start 179.88576 112.703286) (end 179.88576 110.62278) (width 0.75) (layer "B.Cu") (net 20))
 (segment (start 175.966267 116.62278) (end 179.88576 112.703286) (width 0.75) (layer "B.Cu") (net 20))
 (segment (start 173.05076 118.33278) (end 174.76076 116.62278) (width 0.75) (layer "B.Cu") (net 20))
 (segment (start 180.98576 112.94679) (end 180.98576 110.62278) (width 0.75) (layer "B.Cu") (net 21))
 (segment (start 175.59076 118.33278) (end 175.59977 118.33278) (width 0.75) (layer "B.Cu") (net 21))
 (segment (start 175.59977 118.33278) (end 180.98576 112.94679) (width 0.75) (layer "B.Cu") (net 21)))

